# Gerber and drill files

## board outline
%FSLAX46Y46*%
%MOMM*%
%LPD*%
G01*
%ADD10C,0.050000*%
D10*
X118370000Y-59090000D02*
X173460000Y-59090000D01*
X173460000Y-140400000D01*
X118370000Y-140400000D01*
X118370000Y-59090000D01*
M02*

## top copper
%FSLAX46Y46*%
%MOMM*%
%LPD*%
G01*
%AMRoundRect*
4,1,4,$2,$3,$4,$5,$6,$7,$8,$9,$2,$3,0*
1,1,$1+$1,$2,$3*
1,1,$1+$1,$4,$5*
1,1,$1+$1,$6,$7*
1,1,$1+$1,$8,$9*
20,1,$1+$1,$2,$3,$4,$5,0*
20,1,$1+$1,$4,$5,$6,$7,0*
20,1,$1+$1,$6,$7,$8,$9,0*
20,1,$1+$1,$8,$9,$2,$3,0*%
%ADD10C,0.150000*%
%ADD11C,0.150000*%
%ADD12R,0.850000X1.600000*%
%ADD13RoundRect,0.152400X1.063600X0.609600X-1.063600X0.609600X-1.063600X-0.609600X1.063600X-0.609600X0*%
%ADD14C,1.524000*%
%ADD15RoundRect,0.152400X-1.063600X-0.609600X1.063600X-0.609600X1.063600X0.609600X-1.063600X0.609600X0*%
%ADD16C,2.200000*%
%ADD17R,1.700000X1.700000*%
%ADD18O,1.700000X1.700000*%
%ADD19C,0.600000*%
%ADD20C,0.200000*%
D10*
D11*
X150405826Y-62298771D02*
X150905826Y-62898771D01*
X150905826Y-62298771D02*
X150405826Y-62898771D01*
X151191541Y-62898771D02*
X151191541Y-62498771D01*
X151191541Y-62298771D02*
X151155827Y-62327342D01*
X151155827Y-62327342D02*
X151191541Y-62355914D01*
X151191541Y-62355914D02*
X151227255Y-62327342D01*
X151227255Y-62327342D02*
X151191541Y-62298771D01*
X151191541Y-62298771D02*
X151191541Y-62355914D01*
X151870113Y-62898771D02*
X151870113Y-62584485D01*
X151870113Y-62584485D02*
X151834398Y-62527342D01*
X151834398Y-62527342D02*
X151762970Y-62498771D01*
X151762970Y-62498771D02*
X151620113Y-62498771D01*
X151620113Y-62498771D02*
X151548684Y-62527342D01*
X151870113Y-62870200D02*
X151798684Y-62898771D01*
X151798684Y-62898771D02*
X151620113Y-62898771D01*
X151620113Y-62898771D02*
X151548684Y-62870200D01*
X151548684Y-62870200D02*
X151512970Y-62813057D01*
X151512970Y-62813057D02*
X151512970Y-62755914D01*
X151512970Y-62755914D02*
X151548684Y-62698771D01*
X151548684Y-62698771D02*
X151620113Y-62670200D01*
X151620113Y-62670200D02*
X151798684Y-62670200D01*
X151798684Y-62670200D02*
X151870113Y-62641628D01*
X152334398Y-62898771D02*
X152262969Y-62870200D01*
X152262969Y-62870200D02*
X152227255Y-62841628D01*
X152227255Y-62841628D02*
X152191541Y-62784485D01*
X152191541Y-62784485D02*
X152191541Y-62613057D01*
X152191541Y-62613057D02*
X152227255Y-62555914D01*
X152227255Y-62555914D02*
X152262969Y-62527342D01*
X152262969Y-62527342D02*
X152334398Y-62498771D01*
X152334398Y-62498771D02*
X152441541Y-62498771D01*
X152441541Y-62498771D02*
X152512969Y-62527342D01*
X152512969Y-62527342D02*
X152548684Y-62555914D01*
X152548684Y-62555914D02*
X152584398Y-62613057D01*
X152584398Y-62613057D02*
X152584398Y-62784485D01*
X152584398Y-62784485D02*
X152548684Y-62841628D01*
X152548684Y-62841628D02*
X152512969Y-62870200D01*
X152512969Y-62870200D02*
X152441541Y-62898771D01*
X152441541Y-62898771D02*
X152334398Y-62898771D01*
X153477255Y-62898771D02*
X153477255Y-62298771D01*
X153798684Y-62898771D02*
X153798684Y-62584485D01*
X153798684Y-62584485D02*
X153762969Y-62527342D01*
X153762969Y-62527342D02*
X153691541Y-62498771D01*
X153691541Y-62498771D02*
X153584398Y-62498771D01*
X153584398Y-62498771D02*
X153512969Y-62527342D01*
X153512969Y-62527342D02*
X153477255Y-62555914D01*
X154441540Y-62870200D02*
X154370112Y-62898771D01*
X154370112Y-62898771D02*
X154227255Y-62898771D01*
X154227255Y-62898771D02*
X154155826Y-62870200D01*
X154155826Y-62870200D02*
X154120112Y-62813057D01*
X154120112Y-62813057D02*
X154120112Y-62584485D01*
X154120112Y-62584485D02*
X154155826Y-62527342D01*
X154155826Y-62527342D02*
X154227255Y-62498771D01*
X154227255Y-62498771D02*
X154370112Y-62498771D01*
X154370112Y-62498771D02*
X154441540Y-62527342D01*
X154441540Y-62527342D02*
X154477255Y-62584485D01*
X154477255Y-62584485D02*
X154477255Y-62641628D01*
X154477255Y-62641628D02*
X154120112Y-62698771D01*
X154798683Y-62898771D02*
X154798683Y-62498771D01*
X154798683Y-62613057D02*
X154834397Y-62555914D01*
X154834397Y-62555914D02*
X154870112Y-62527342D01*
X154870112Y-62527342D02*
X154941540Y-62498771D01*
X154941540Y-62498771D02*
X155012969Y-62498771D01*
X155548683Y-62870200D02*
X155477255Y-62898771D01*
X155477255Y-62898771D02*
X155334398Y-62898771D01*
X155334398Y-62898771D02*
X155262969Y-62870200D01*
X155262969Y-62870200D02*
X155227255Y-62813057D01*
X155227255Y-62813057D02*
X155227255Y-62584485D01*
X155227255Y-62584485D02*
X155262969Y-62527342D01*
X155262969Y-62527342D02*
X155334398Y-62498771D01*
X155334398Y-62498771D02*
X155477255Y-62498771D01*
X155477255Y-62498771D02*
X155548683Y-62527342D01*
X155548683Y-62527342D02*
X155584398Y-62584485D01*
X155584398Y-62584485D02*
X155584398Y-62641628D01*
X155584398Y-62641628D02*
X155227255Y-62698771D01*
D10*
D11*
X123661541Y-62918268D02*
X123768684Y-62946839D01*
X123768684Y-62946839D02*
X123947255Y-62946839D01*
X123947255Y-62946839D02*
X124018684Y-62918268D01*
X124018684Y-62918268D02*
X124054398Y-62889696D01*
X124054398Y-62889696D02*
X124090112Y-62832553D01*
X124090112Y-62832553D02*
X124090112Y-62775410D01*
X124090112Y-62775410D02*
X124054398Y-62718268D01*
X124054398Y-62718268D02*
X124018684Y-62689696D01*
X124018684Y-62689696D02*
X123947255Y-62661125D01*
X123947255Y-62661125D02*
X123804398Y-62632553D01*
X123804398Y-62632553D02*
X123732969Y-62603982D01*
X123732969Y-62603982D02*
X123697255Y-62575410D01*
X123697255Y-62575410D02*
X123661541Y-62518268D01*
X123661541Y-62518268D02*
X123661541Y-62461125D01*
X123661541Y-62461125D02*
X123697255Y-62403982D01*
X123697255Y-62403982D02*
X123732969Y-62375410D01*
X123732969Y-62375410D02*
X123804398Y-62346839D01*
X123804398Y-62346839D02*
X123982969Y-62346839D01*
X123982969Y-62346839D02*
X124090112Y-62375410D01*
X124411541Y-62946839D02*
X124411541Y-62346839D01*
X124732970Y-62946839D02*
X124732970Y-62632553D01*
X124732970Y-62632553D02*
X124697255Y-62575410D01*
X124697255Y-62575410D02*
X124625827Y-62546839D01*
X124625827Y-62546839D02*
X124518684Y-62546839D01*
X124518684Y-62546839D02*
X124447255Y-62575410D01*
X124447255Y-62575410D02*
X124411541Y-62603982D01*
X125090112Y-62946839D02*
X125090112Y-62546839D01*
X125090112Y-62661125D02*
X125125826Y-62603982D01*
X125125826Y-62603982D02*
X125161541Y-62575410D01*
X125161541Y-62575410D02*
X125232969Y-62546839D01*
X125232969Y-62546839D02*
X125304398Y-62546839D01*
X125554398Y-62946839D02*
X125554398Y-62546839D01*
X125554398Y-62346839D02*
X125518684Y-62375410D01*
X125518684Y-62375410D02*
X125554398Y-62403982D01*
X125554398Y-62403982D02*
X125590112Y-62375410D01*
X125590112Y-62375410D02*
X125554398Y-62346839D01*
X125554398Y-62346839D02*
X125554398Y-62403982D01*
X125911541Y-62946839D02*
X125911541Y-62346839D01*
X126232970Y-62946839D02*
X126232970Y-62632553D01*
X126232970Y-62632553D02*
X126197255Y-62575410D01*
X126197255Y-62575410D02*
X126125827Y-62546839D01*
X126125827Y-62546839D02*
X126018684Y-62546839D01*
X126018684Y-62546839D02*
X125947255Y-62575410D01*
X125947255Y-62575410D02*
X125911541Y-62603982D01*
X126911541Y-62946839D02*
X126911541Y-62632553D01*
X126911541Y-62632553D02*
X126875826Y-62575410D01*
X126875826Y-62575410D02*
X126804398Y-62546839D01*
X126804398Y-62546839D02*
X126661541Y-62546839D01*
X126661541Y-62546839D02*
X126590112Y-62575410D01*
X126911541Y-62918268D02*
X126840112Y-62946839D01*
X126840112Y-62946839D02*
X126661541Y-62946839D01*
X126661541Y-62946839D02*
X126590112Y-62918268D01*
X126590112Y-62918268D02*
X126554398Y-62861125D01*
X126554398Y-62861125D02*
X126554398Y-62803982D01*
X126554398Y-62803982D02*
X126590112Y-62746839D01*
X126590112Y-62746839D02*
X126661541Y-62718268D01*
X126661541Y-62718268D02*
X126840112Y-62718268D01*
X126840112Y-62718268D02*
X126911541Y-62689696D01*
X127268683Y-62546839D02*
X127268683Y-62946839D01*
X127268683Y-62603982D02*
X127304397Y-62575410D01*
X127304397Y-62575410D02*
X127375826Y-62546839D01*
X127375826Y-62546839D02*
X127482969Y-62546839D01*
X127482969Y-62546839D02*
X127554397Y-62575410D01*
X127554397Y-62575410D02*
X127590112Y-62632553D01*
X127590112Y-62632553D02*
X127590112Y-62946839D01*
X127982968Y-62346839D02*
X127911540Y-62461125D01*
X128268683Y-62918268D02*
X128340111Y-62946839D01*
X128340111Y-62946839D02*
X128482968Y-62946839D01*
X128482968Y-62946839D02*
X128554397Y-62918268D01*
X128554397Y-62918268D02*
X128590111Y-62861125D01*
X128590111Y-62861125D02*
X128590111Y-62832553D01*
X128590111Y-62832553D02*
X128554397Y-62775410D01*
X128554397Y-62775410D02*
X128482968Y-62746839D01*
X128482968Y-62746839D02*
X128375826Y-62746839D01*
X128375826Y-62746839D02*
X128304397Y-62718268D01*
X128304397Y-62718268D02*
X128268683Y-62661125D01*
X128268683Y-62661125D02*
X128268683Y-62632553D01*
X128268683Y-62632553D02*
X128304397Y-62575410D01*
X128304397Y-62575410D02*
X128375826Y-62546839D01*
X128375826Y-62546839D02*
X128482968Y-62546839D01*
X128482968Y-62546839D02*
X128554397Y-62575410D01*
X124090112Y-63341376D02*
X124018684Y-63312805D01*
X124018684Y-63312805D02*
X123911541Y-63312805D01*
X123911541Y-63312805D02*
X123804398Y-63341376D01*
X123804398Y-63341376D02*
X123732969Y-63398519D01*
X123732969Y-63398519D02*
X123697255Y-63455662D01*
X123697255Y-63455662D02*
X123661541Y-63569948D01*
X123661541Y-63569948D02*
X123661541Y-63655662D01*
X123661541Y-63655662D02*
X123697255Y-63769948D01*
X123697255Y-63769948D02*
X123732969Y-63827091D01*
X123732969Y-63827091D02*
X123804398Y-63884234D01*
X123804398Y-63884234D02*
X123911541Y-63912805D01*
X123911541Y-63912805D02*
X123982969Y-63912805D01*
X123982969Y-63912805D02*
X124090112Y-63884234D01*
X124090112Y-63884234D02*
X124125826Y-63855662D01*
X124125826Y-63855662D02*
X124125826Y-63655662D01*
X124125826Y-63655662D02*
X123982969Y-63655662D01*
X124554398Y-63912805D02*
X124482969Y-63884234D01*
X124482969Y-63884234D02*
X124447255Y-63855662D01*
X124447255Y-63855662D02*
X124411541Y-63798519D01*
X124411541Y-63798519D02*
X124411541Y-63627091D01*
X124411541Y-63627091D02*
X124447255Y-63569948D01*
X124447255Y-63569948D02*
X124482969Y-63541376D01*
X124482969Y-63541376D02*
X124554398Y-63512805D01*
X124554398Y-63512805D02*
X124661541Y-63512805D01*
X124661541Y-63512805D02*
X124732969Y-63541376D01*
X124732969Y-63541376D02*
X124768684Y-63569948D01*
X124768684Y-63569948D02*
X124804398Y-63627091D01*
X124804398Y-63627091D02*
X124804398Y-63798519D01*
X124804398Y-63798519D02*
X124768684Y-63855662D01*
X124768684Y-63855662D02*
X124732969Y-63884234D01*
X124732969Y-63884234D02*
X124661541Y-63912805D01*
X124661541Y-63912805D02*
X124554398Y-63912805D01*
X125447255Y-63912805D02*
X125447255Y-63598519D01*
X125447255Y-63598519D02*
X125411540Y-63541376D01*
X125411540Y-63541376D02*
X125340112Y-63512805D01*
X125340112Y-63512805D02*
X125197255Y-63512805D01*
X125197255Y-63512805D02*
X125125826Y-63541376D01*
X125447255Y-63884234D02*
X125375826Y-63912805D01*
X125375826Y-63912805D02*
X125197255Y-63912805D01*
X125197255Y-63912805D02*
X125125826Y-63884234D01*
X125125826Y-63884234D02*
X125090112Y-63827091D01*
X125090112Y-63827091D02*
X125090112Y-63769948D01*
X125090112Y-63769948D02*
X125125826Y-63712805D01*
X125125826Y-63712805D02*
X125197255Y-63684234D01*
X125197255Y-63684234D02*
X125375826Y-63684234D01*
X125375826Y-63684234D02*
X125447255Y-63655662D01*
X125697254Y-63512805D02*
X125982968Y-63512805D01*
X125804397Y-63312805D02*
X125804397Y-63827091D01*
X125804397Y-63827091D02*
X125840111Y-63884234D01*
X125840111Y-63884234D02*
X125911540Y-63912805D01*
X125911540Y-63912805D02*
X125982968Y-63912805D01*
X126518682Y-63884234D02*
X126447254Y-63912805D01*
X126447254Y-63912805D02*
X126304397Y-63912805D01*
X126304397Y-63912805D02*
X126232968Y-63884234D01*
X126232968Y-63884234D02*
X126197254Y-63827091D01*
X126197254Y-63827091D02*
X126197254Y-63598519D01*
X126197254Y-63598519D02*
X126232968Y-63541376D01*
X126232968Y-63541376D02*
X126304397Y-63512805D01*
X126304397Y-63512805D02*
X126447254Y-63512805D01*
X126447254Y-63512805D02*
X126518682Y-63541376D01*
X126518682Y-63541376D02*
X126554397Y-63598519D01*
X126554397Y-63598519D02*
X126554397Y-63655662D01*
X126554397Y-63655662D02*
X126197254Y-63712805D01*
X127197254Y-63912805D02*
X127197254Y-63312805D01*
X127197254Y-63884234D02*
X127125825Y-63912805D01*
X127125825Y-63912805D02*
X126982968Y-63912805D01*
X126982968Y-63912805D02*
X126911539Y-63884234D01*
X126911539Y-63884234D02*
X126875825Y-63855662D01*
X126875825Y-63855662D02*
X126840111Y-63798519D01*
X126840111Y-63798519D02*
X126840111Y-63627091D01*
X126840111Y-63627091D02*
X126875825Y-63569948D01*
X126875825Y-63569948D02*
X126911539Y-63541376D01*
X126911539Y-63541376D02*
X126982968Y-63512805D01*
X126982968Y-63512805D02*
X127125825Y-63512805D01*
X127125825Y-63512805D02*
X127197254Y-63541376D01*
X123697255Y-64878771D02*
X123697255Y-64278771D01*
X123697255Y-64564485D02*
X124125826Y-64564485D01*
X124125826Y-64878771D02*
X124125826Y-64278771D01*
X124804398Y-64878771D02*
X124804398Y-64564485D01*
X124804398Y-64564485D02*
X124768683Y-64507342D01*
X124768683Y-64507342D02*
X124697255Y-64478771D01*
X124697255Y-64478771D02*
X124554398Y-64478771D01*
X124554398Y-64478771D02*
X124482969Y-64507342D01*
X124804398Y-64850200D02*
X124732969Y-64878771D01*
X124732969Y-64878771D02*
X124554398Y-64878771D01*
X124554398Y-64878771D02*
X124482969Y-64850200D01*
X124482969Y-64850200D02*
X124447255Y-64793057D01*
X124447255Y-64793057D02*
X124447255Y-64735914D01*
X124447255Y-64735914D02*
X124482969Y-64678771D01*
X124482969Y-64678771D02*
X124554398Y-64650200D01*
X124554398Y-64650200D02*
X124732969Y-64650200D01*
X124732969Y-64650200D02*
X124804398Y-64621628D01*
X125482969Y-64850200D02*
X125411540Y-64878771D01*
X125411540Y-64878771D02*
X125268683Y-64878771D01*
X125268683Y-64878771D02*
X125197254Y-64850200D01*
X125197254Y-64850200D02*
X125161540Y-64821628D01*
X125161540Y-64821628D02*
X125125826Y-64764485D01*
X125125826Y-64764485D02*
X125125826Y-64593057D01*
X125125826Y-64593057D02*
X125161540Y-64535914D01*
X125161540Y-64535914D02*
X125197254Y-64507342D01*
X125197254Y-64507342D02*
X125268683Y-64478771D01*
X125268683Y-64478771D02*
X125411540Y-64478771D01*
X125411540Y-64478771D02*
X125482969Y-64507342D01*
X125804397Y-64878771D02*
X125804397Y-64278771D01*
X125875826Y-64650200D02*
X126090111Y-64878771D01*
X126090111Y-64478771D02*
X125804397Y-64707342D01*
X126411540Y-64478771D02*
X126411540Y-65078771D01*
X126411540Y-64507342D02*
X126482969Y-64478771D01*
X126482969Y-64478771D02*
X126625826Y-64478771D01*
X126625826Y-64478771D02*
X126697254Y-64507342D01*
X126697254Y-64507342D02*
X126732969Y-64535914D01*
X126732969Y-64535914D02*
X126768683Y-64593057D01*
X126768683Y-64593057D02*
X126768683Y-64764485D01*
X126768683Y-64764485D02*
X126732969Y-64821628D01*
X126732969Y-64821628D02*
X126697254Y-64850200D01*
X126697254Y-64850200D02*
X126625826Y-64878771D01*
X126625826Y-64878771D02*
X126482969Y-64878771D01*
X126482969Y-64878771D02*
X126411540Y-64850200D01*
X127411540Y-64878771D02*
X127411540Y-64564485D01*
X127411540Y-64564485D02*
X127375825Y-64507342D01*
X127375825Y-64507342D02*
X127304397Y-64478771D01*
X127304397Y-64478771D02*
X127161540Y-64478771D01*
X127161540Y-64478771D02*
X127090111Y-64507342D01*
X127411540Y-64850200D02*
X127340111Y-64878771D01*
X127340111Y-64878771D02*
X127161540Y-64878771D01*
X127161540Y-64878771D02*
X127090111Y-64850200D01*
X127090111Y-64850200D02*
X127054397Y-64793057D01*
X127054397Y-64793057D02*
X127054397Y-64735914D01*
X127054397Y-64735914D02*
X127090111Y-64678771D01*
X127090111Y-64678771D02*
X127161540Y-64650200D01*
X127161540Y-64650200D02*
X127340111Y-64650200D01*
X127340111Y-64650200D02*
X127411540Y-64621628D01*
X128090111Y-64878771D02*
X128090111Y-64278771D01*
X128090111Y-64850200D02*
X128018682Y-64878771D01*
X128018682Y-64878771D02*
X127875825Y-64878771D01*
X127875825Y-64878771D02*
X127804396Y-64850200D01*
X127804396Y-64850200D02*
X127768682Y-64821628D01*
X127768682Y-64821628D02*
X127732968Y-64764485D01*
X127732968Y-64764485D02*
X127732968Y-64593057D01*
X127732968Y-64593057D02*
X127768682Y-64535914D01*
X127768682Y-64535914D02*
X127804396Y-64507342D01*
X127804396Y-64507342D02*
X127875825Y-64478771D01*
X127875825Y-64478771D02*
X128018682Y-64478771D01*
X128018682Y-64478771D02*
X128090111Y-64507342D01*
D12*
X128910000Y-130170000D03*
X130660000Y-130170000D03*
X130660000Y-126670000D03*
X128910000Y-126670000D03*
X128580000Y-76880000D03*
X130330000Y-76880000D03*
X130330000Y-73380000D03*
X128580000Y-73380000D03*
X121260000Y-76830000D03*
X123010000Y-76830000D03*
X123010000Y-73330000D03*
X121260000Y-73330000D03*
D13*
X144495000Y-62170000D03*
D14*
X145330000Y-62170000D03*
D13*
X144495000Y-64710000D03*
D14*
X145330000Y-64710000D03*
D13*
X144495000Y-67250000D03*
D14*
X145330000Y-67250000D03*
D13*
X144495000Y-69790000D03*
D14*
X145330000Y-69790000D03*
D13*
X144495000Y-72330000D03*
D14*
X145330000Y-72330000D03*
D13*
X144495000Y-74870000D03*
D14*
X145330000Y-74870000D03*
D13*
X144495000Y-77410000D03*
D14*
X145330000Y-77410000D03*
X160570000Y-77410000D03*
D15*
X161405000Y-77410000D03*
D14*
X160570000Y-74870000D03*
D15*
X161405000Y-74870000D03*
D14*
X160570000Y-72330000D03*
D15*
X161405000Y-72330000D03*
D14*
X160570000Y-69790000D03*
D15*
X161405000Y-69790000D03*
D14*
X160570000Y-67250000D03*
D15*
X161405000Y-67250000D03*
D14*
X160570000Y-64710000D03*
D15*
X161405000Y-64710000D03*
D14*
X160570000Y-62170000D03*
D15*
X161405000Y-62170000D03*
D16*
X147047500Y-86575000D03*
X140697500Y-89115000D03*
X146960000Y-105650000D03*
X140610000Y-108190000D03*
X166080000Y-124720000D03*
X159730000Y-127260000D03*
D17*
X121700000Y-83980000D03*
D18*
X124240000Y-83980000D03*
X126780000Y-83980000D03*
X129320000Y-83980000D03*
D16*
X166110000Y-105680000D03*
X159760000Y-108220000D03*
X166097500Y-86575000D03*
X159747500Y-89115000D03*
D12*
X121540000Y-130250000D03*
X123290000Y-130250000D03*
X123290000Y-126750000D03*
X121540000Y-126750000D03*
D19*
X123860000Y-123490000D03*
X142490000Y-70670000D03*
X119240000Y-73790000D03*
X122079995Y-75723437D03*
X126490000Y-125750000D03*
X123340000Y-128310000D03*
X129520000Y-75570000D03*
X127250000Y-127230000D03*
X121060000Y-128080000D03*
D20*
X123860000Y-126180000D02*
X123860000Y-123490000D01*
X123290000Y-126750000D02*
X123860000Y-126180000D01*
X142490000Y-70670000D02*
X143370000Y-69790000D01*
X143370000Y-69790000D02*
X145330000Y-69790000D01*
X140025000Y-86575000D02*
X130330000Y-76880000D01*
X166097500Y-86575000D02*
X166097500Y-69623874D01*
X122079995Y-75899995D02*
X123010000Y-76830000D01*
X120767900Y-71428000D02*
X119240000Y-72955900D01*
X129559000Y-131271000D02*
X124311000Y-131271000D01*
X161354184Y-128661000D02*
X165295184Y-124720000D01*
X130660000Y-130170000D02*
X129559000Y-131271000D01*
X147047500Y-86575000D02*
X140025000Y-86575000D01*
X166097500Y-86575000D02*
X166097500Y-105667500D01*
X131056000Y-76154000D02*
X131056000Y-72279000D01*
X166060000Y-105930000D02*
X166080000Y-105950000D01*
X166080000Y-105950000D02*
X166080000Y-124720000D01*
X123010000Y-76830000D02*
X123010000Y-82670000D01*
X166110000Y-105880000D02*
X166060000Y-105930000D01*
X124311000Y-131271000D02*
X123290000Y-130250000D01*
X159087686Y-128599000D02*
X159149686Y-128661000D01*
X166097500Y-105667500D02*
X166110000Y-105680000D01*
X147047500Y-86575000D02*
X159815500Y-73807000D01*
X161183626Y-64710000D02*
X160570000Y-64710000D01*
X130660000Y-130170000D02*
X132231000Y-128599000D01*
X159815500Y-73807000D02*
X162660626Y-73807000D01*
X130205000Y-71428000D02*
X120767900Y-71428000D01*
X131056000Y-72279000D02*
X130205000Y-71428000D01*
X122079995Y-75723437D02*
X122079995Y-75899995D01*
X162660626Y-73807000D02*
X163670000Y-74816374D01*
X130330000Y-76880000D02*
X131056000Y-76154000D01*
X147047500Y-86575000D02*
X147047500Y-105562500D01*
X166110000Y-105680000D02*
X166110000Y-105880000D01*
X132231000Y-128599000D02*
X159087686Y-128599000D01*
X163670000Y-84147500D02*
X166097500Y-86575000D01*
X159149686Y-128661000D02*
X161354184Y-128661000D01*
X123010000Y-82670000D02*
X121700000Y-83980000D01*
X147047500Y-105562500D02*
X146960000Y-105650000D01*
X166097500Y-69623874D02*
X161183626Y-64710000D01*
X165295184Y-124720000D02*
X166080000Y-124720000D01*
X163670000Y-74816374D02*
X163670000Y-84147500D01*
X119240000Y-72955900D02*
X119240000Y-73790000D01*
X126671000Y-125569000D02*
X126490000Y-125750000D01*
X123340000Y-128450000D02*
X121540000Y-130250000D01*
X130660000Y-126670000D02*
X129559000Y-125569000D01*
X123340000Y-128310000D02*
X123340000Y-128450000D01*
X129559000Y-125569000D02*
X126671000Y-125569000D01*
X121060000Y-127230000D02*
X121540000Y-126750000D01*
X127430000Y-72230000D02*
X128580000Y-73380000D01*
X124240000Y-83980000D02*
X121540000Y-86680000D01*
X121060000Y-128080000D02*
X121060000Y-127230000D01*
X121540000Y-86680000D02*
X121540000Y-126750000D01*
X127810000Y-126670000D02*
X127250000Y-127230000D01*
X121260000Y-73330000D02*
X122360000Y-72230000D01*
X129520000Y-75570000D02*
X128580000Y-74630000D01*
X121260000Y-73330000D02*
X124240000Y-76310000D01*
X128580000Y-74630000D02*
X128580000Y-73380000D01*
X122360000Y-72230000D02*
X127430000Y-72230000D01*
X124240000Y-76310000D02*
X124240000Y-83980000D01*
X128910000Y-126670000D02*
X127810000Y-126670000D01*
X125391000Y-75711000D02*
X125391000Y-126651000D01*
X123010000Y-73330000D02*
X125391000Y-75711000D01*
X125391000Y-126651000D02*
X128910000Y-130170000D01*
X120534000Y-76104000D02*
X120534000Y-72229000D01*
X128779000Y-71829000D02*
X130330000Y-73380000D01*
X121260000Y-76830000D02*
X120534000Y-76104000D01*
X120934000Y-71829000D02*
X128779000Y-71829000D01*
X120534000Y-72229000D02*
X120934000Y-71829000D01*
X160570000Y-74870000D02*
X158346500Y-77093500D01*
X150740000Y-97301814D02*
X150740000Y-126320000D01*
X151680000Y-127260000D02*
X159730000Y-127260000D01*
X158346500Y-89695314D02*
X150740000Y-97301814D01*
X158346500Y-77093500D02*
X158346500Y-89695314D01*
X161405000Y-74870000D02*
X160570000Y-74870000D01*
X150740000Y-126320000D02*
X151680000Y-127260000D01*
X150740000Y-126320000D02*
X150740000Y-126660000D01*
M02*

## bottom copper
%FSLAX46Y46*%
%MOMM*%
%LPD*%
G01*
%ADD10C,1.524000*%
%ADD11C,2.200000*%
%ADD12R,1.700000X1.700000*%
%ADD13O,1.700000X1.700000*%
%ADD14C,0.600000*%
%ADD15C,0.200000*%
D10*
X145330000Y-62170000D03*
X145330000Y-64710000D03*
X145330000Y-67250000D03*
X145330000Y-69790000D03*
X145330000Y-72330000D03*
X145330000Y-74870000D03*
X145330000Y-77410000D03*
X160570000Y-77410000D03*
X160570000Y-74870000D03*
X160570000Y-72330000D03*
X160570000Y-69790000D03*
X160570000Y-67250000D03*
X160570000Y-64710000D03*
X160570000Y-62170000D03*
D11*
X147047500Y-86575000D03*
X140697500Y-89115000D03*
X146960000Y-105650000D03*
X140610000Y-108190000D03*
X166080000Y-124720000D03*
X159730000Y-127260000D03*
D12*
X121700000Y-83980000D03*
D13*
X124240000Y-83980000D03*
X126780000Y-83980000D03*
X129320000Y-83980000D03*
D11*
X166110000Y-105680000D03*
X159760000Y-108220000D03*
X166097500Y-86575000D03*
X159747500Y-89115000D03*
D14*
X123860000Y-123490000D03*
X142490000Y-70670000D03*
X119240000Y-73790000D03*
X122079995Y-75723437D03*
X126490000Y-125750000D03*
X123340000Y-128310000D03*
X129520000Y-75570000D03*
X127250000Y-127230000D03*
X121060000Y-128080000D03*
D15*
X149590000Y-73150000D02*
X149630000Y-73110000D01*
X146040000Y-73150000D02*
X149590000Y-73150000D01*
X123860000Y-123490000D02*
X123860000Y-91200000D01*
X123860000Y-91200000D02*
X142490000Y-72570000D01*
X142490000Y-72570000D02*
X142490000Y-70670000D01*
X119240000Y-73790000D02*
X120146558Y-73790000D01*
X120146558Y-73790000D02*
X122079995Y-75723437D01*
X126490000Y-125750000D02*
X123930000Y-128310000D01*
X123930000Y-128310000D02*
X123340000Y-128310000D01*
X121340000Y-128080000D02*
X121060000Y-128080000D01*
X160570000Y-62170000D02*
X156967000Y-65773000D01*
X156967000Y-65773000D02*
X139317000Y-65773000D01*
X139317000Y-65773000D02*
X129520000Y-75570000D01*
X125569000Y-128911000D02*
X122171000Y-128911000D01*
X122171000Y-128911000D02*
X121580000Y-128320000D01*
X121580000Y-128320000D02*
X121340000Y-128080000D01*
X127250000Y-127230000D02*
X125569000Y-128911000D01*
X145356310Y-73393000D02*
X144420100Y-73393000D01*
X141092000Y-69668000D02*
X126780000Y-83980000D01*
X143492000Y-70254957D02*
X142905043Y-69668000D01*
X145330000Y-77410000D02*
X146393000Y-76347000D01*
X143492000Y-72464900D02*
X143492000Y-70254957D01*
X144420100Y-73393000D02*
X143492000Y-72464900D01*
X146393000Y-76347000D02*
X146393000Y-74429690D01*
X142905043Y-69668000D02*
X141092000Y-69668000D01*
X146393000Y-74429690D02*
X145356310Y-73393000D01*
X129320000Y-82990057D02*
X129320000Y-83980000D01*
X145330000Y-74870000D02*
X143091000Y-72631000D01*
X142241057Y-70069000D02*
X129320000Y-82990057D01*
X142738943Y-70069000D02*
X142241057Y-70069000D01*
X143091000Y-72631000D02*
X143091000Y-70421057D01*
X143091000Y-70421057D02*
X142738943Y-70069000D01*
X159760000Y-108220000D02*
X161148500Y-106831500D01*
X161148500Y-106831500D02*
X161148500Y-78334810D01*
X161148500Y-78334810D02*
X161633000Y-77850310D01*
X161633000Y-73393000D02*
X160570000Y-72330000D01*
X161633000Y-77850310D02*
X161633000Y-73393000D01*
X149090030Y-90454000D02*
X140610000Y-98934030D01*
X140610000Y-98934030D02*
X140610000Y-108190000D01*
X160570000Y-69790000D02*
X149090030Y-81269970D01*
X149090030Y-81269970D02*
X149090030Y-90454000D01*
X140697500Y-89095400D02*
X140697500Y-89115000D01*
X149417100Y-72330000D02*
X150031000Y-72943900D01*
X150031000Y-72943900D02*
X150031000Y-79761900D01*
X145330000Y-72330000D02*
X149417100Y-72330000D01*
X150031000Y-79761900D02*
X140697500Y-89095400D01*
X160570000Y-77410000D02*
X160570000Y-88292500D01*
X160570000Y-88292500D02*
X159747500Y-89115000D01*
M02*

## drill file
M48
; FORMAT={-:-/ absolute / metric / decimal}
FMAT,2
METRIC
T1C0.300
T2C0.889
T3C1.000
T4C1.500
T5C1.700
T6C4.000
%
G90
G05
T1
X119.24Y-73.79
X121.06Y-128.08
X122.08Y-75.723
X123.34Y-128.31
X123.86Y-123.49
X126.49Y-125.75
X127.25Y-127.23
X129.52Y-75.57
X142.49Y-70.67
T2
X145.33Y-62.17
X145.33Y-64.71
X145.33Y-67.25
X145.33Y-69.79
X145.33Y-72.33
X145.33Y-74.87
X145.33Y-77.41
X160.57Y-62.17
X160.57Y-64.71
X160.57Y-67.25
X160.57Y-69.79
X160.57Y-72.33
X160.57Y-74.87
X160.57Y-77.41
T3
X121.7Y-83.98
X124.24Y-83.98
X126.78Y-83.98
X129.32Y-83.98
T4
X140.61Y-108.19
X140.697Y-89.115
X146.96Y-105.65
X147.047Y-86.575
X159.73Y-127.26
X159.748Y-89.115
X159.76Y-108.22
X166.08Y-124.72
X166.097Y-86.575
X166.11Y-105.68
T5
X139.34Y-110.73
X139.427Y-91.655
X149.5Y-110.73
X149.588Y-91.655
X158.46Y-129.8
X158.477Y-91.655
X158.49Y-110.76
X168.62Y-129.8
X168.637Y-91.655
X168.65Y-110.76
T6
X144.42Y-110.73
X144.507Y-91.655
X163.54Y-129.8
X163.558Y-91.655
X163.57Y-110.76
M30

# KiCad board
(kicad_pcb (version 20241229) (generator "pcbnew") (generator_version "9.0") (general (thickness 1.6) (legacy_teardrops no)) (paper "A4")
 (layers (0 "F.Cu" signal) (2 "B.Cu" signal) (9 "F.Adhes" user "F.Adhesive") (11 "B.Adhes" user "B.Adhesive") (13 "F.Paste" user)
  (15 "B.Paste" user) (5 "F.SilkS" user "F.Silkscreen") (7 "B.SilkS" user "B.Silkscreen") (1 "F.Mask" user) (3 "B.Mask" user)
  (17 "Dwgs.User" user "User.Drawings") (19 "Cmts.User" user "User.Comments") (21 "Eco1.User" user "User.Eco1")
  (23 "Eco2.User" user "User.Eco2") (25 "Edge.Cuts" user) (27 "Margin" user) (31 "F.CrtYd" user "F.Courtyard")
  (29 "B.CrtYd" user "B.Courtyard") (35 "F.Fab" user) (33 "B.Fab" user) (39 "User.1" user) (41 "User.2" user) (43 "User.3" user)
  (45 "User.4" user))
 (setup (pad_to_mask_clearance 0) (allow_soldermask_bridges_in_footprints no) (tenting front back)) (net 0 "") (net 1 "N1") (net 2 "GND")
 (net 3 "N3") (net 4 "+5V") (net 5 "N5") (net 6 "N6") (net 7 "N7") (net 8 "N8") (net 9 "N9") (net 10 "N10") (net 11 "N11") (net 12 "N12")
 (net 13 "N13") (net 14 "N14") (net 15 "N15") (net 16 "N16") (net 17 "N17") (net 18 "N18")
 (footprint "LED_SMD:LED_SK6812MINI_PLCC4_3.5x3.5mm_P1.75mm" (layer "F.Cu") (at 129.785 128.42 90)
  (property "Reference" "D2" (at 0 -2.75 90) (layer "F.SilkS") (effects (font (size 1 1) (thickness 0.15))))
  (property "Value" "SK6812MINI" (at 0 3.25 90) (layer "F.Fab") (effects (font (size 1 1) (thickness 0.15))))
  (pad "1" smd rect (at -1.75 -0.875 90) (size 1.6 0.85) (layers "F.Cu" "F.Mask" "F.Paste") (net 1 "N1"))
  (pad "2" smd rect (at -1.75 0.875 90) (size 1.6 0.85) (layers "F.Cu" "F.Mask" "F.Paste") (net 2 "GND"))
  (pad "3" smd rect (at 1.75 0.875 90) (size 1.6 0.85) (layers "F.Cu" "F.Mask" "F.Paste") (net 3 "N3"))
  (pad "4" smd rect (at 1.75 -0.875 90) (size 1.6 0.85) (layers "F.Cu" "F.Mask" "F.Paste") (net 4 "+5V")))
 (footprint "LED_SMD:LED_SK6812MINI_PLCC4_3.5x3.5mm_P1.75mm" (layer "F.Cu") (at 129.455 75.13 90)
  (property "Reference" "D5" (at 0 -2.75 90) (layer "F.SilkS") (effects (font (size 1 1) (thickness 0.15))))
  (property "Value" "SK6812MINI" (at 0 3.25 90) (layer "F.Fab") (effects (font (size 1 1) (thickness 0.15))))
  (pad "1" smd rect (at -1.75 -0.875 90) (size 1.6 0.85) (layers "F.Cu" "F.Mask" "F.Paste") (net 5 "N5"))
  (pad "2" smd rect (at -1.75 0.875 90) (size 1.6 0.85) (layers "F.Cu" "F.Mask" "F.Paste") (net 2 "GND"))
  (pad "3" smd rect (at 1.75 0.875 90) (size 1.6 0.85) (layers "F.Cu" "F.Mask" "F.Paste") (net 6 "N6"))
  (pad "4" smd rect (at 1.75 -0.875 90) (size 1.6 0.85) (layers "F.Cu" "F.Mask" "F.Paste") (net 4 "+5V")))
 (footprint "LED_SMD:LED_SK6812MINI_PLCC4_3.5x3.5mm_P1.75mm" (layer "F.Cu") (at 122.135 75.08 90)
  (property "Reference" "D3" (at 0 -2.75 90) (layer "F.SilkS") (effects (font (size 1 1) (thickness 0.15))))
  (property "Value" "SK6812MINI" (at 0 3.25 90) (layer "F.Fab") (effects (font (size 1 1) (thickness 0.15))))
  (pad "1" smd rect (at -1.75 -0.875 90) (size 1.6 0.85) (layers "F.Cu" "F.Mask" "F.Paste") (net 6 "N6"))
  (pad "2" smd rect (at -1.75 0.875 90) (size 1.6 0.85) (layers "F.Cu" "F.Mask" "F.Paste") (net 2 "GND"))
  (pad "3" smd rect (at 1.75 0.875 90) (size 1.6 0.85) (layers "F.Cu" "F.Mask" "F.Paste") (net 1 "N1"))
  (pad "4" smd rect (at 1.75 -0.875 90) (size 1.6 0.85) (layers "F.Cu" "F.Mask" "F.Paste") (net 4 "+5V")))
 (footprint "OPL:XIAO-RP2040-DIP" (layer "F.Cu") (at 152.95 69.79)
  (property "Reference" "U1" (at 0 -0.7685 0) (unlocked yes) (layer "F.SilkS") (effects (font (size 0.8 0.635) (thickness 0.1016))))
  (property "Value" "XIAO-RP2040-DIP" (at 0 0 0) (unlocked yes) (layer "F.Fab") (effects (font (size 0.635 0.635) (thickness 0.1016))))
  (pad "1" smd roundrect (at -8.455 -7.62 180) (size 2.432 1.524) (layers "F.Cu" "F.Mask") (roundrect_rratio 0.1) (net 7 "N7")
   (thermal_bridge_angle 45))
  (pad "1" thru_hole circle (at -7.62 -7.62 180) (size 1.524 1.524) (drill 0.889) (layers "*.Cu" "*.Mask") (remove_unused_layers no)
   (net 7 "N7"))
  (pad "2" smd roundrect (at -8.455 -5.08 180) (size 2.432 1.524) (layers "F.Cu" "F.Mask") (roundrect_rratio 0.1) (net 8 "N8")
   (thermal_bridge_angle 45))
  (pad "2" thru_hole circle (at -7.62 -5.08 180) (size 1.524 1.524) (drill 0.889) (layers "*.Cu" "*.Mask") (remove_unused_layers no)
   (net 8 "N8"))
  (pad "3" smd roundrect (at -8.455 -2.54 180) (size 2.432 1.524) (layers "F.Cu" "F.Mask") (roundrect_rratio 0.1) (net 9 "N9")
   (thermal_bridge_angle 45))
  (pad "3" thru_hole circle (at -7.62 -2.54 180) (size 1.524 1.524) (drill 0.889) (layers "*.Cu" "*.Mask") (remove_unused_layers no)
   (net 9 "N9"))
  (pad "4" smd roundrect (at -8.455 0 180) (size 2.432 1.524) (layers "F.Cu" "F.Mask") (roundrect_rratio 0.1) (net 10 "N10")
   (thermal_bridge_angle 45))
  (pad "4" thru_hole circle (at -7.62 0 180) (size 1.524 1.524) (drill 0.889) (layers "*.Cu" "*.Mask") (remove_unused_layers no)
   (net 10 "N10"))
  (pad "5" smd roundrect (at -8.455 2.54 180) (size 2.432 1.524) (layers "F.Cu" "F.Mask") (roundrect_rratio 0.1) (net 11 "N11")
   (thermal_bridge_angle 45))
  (pad "5" thru_hole circle (at -7.62 2.54 180) (size 1.524 1.524) (drill 0.889) (layers "*.Cu" "*.Mask") (remove_unused_layers no)
   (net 11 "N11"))
  (pad "6" smd roundrect (at -8.455 5.08 180) (size 2.432 1.524) (layers "F.Cu" "F.Mask") (roundrect_rratio 0.1) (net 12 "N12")
   (thermal_bridge_angle 45))
  (pad "6" thru_hole circle (at -7.62 5.08 180) (size 1.524 1.524) (drill 0.889) (layers "*.Cu" "*.Mask") (remove_unused_layers no)
   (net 12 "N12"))
  (pad "7" smd roundrect (at -8.455 7.62 180) (size 2.432 1.524) (layers "F.Cu" "F.Mask") (roundrect_rratio 0.1) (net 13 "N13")
   (thermal_bridge_angle 45))
  (pad "7" thru_hole circle (at -7.62 7.62 180) (size 1.524 1.524) (drill 0.889) (layers "*.Cu" "*.Mask") (remove_unused_layers no)
   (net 13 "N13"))
  (pad "8" thru_hole circle (at 7.62 7.62) (size 1.524 1.524) (drill 0.889) (layers "*.Cu" "*.Mask") (remove_unused_layers no)
   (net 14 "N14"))
  (pad "8" smd roundrect (at 8.455 7.62) (size 2.432 1.524) (layers "F.Cu" "F.Mask") (roundrect_rratio 0.1) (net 14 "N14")
   (thermal_bridge_angle 45))
  (pad "9" thru_hole circle (at 7.62 5.08) (size 1.524 1.524) (drill 0.889) (layers "*.Cu" "*.Mask") (remove_unused_layers no)
   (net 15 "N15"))
  (pad "9" smd roundrect (at 8.455 5.08) (size 2.432 1.524) (layers "F.Cu" "F.Mask") (roundrect_rratio 0.1) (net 15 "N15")
   (thermal_bridge_angle 45))
  (pad "10" thru_hole circle (at 7.62 2.54) (size 1.524 1.524) (drill 0.889) (layers "*.Cu" "*.Mask") (remove_unused_layers no)
   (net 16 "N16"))
  (pad "10" smd roundrect (at 8.455 2.54) (size 2.432 1.524) (layers "F.Cu" "F.Mask") (roundrect_rratio 0.1) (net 16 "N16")
   (thermal_bridge_angle 45))
  (pad "11" thru_hole circle (at 7.62 0) (size 1.524 1.524) (drill 0.889) (layers "*.Cu" "*.Mask") (remove_unused_layers no) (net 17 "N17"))
  (pad "11" smd roundrect (at 8.455 0) (size 2.432 1.524) (layers "F.Cu" "F.Mask") (roundrect_rratio 0.1) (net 17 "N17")
   (thermal_bridge_angle 45))
  (pad "12" thru_hole circle (at 7.62 -2.54) (size 1.524 1.524) (drill 0.889) (layers "*.Cu" "*.Mask") (remove_unused_layers no)
   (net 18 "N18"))
  (pad "12" smd roundrect (at 8.455 -2.54) (size 2.432 1.524) (layers "F.Cu" "F.Mask") (roundrect_rratio 0.1) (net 18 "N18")
   (thermal_bridge_angle 45))
  (pad "13" thru_hole circle (at 7.62 -5.08) (size 1.524 1.524) (drill 0.889) (layers "*.Cu" "*.Mask") (remove_unused_layers no)
   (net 2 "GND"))
  (pad "13" smd roundrect (at 8.455 -5.08) (size 2.432 1.524) (layers "F.Cu" "F.Mask") (roundrect_rratio 0.1) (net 2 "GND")
   (thermal_bridge_angle 45))
  (pad "14" thru_hole circle (at 7.62 -7.62) (size 1.524 1.524) (drill 0.889) (layers "*.Cu" "*.Mask") (remove_unused_layers no)
   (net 4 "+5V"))
  (pad "14" smd roundrect (at 8.455 -7.62) (size 2.432 1.524) (layers "F.Cu" "F.Mask") (roundrect_rratio 0.1) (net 4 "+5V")
   (thermal_bridge_angle 45)))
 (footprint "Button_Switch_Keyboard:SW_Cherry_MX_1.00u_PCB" (layer "F.Cu") (at 147.0475 86.575)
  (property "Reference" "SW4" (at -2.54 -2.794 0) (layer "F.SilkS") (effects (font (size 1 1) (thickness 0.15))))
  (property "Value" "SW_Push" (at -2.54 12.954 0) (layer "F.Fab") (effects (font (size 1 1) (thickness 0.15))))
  (pad "" np_thru_hole circle (at -7.62 5.08) (size 1.7 1.7) (drill 1.7) (layers "*.Cu" "*.Mask"))
  (pad "" np_thru_hole circle (at -2.54 5.08) (size 4 4) (drill 4) (layers "*.Cu" "*.Mask"))
  (pad "" np_thru_hole circle (at 2.54 5.08) (size 1.7 1.7) (drill 1.7) (layers "*.Cu" "*.Mask"))
  (pad "1" thru_hole circle (at 0 0) (size 2.2 2.2) (drill 1.5) (layers "*.Cu" "*.Mask") (remove_unused_layers no) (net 2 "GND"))
  (pad "2" thru_hole circle (at -6.35 2.54) (size 2.2 2.2) (drill 1.5) (layers "*.Cu" "*.Mask") (remove_unused_layers no) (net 11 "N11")))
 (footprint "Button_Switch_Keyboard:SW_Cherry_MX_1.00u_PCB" (layer "F.Cu") (at 146.96 105.65)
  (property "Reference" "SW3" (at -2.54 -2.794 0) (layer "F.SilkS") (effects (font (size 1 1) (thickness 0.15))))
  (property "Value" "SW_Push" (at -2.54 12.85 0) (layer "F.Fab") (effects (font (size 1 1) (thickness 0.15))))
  (pad "" np_thru_hole circle (at -7.62 5.08) (size 1.7 1.7) (drill 1.7) (layers "*.Cu" "*.Mask"))
  (pad "" np_thru_hole circle (at -2.54 5.08) (size 4 4) (drill 4) (layers "*.Cu" "*.Mask"))
  (pad "" np_thru_hole circle (at 2.54 5.08) (size 1.7 1.7) (drill 1.7) (layers "*.Cu" "*.Mask"))
  (pad "1" thru_hole circle (at 0 0) (size 2.2 2.2) (drill 1.5) (layers "*.Cu" "*.Mask") (remove_unused_layers no) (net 2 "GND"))
  (pad "2" thru_hole circle (at -6.35 2.54) (size 2.2 2.2) (drill 1.5) (layers "*.Cu" "*.Mask") (remove_unused_layers no) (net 17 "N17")))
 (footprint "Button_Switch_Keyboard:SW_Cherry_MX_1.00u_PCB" (layer "F.Cu") (at 166.08 124.72)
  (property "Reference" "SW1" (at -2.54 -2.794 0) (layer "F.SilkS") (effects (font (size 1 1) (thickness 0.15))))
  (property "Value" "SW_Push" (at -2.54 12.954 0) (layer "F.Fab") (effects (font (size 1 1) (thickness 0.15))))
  (pad "" np_thru_hole circle (at -7.62 5.08) (size 1.7 1.7) (drill 1.7) (layers "*.Cu" "*.Mask"))
  (pad "" np_thru_hole circle (at -2.54 5.08) (size 4 4) (drill 4) (layers "*.Cu" "*.Mask"))
  (pad "" np_thru_hole circle (at 2.54 5.08) (size 1.7 1.7) (drill 1.7) (layers "*.Cu" "*.Mask"))
  (pad "1" thru_hole circle (at 0 0) (size 2.2 2.2) (drill 1.5) (layers "*.Cu" "*.Mask") (remove_unused_layers no) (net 2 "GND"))
  (pad "2" thru_hole circle (at -6.35 2.54) (size 2.2 2.2) (drill 1.5) (layers "*.Cu" "*.Mask") (remove_unused_layers no) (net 15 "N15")))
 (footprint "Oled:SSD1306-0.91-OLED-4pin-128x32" (layer "F.Cu") (at 119.51 120.48 90)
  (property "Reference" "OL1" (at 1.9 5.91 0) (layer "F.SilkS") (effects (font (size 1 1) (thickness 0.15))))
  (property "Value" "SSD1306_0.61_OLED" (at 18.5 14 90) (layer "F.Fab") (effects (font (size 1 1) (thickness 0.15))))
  (pad "1" thru_hole rect (at 36.5 2.19 90) (size 1.7 1.7) (drill 1) (layers "*.Cu" "*.Mask") (remove_unused_layers no) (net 2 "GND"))
  (pad "2" thru_hole oval (at 36.5 4.73 90) (size 1.7 1.7) (drill 1) (layers "*.Cu" "*.Mask") (remove_unused_layers no) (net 4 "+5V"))
  (pad "3" thru_hole oval (at 36.5 7.27 90) (size 1.7 1.7) (drill 1) (layers "*.Cu" "*.Mask") (remove_unused_layers no) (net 13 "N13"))
  (pad "4" thru_hole oval (at 36.5 9.81 90) (size 1.7 1.7) (drill 1) (layers "*.Cu" "*.Mask") (remove_unused_layers no) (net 12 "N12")))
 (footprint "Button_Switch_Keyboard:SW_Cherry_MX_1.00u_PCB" (layer "F.Cu") (at 166.11 105.68)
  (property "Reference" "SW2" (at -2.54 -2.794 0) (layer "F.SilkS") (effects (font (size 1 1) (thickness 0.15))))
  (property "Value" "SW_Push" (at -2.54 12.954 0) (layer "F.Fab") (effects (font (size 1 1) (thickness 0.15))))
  (pad "" np_thru_hole circle (at -7.62 5.08) (size 1.7 1.7) (drill 1.7) (layers "*.Cu" "*.Mask"))
  (pad "" np_thru_hole circle (at -2.54 5.08) (size 4 4) (drill 4) (layers "*.Cu" "*.Mask"))
  (pad "" np_thru_hole circle (at 2.54 5.08) (size 1.7 1.7) (drill 1.7) (layers "*.Cu" "*.Mask"))
  (pad "1" thru_hole circle (at 0 0) (size 2.2 2.2) (drill 1.5) (layers "*.Cu" "*.Mask") (remove_unused_layers no) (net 2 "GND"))
  (pad "2" thru_hole circle (at -6.35 2.54) (size 2.2 2.2) (drill 1.5) (layers "*.Cu" "*.Mask") (remove_unused_layers no) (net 16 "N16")))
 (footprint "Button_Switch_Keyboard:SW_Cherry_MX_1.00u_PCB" (layer "F.Cu") (at 166.0975 86.575)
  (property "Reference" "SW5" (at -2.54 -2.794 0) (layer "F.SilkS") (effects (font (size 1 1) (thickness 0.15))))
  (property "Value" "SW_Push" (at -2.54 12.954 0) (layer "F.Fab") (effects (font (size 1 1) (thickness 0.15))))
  (pad "" np_thru_hole circle (at -7.62 5.08) (size 1.7 1.7) (drill 1.7) (layers "*.Cu" "*.Mask"))
  (pad "" np_thru_hole circle (at -2.54 5.08) (size 4 4) (drill 4) (layers "*.Cu" "*.Mask"))
  (pad "" np_thru_hole circle (at 2.54 5.08) (size 1.7 1.7) (drill 1.7) (layers "*.Cu" "*.Mask"))
  (pad "1" thru_hole circle (at 0 0) (size 2.2 2.2) (drill 1.5) (layers "*.Cu" "*.Mask") (remove_unused_layers no) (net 2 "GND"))
  (pad "2" thru_hole circle (at -6.35 2.54) (size 2.2 2.2) (drill 1.5) (layers "*.Cu" "*.Mask") (remove_unused_layers no) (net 14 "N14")))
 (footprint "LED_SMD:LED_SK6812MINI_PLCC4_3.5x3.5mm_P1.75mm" (layer "F.Cu") (at 122.415 128.5 90)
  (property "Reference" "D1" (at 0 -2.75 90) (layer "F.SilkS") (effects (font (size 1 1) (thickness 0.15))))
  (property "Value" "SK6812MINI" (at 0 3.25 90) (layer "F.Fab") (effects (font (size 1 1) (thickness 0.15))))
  (pad "1" smd rect (at -1.75 -0.875 90) (size 1.6 0.85) (layers "F.Cu" "F.Mask" "F.Paste") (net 3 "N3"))
  (pad "2" smd rect (at -1.75 0.875 90) (size 1.6 0.85) (layers "F.Cu" "F.Mask" "F.Paste") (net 2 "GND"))
  (pad "3" smd rect (at 1.75 0.875 90) (size 1.6 0.85) (layers "F.Cu" "F.Mask" "F.Paste") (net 10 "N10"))
  (pad "4" smd rect (at 1.75 -0.875 90) (size 1.6 0.85) (layers "F.Cu" "F.Mask" "F.Paste") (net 4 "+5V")))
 (gr_rect (start 118.37 59.09) (end 173.46 140.4) (stroke (width 0.05) (type default)) (fill no) (layer "Edge.Cuts"))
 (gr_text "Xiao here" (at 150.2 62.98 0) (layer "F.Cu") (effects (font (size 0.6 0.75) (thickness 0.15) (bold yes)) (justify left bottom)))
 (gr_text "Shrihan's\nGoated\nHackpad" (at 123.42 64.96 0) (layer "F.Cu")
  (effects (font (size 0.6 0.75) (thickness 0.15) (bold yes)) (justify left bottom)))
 (segment (start 149.59 73.15) (end 149.63 73.11) (width 0.2) (layer "B.Cu") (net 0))
 (segment (start 146.04 73.15) (end 149.59 73.15) (width 0.2) (layer "B.Cu") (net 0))
 (segment (start 123.86 126.18) (end 123.86 123.49) (width 0.2) (layer "F.Cu") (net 10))
 (segment (start 123.29 126.75) (end 123.86 126.18) (width 0.2) (layer "F.Cu") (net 10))
 (segment (start 142.49 70.67) (end 143.37 69.79) (width 0.2) (layer "F.Cu") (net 10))
 (segment (start 143.37 69.79) (end 145.33 69.79) (width 0.2) (layer "F.Cu") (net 10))
 (via (at 123.86 123.49) (size 0.6) (drill 0.3) (layers "F.Cu" "B.Cu") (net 10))
 (via (at 142.49 70.67) (size 0.6) (drill 0.3) (layers "F.Cu" "B.Cu") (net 10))
 (segment (start 123.86 123.49) (end 123.86 91.2) (width 0.2) (layer "B.Cu") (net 10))
 (segment (start 123.86 91.2) (end 142.49 72.57) (width 0.2) (layer "B.Cu") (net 10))
 (segment (start 142.49 72.57) (end 142.49 70.67) (width 0.2) (layer "B.Cu") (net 10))
 (segment (start 140.025 86.575) (end 130.33 76.88) (width 0.2) (layer "F.Cu") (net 2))
 (segment (start 166.0975 86.575) (end 166.0975 69.623874) (width 0.2) (layer "F.Cu") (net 2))
 (segment (start 122.079995 75.899995) (end 123.01 76.83) (width 0.2) (layer "F.Cu") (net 2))
 (segment (start 120.7679 71.428) (end 119.24 72.9559) (width 0.2) (layer "F.Cu") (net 2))
 (segment (start 129.559 131.271) (end 124.311 131.271) (width 0.2) (layer "F.Cu") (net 2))
 (segment (start 161.354184 128.661) (end 165.295184 124.72) (width 0.2) (layer "F.Cu") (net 2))
 (segment (start 130.66 130.17) (end 129.559 131.271) (width 0.2) (layer "F.Cu") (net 2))
 (segment (start 147.0475 86.575) (end 140.025 86.575) (width 0.2) (layer "F.Cu") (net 2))
 (segment (start 166.0975 86.575) (end 166.0975 105.6675) (width 0.2) (layer "F.Cu") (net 2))
 (segment (start 131.056 76.154) (end 131.056 72.279) (width 0.2) (layer "F.Cu") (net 2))
 (segment (start 166.06 105.93) (end 166.08 105.95) (width 0.2) (layer "F.Cu") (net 2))
 (segment (start 166.08 105.95) (end 166.08 124.72) (width 0.2) (layer "F.Cu") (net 2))
 (segment (start 123.01 76.83) (end 123.01 82.67) (width 0.2) (layer "F.Cu") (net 2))
 (segment (start 166.11 105.88) (end 166.06 105.93) (width 0.2) (layer "F.Cu") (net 2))
 (segment (start 124.311 131.271) (end 123.29 130.25) (width 0.2) (layer "F.Cu") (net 2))
 (segment (start 159.087686 128.599) (end 159.149686 128.661) (width 0.2) (layer "F.Cu") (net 2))
 (segment (start 166.0975 105.6675) (end 166.11 105.68) (width 0.2) (layer "F.Cu") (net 2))
 (segment (start 147.0475 86.575) (end 159.8155 73.807) (width 0.2) (layer "F.Cu") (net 2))
 (segment (start 161.183626 64.71) (end 160.57 64.71) (width 0.2) (layer "F.Cu") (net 2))
 (segment (start 130.66 130.17) (end 132.231 128.599) (width 0.2) (layer "F.Cu") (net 2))
 (segment (start 159.8155 73.807) (end 162.660626 73.807) (width 0.2) (layer "F.Cu") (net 2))
 (segment (start 130.205 71.428) (end 120.7679 71.428) (width 0.2) (layer "F.Cu") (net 2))
 (segment (start 131.056 72.279) (end 130.205 71.428) (width 0.2) (layer "F.Cu") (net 2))
 (segment (start 122.079995 75.723437) (end 122.079995 75.899995) (width 0.2) (layer "F.Cu") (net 2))
 (segment (start 162.660626 73.807) (end 163.67 74.816374) (width 0.2) (layer "F.Cu") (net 2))
 (segment (start 130.33 76.88) (end 131.056 76.154) (width 0.2) (layer "F.Cu") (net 2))
 (segment (start 147.0475 86.575) (end 147.0475 105.5625) (width 0.2) (layer "F.Cu") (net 2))
 (segment (start 166.11 105.68) (end 166.11 105.88) (width 0.2) (layer "F.Cu") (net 2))
 (segment (start 132.231 128.599) (end 159.087686 128.599) (width 0.2) (layer "F.Cu") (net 2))
 (segment (start 163.67 84.1475) (end 166.0975 86.575) (width 0.2) (layer "F.Cu") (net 2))
 (segment (start 159.149686 128.661) (end 161.354184 128.661) (width 0.2) (layer "F.Cu") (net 2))
 (segment (start 123.01 82.67) (end 121.7 83.98) (width 0.2) (layer "F.Cu") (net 2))
 (segment (start 147.0475 105.5625) (end 146.96 105.65) (width 0.2) (layer "F.Cu") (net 2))
 (segment (start 166.0975 69.623874) (end 161.183626 64.71) (width 0.2) (layer "F.Cu") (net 2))
 (segment (start 165.295184 124.72) (end 166.08 124.72) (width 0.2) (layer "F.Cu") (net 2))
 (segment (start 163.67 74.816374) (end 163.67 84.1475) (width 0.2) (layer "F.Cu") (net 2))
 (segment (start 119.24 72.9559) (end 119.24 73.79) (width 0.2) (layer "F.Cu") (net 2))
 (via (at 119.24 73.79) (size 0.6) (drill 0.3) (layers "F.Cu" "B.Cu") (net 2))
 (via (at 122.079995 75.723437) (size 0.6) (drill 0.3) (layers "F.Cu" "B.Cu") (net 2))
 (segment (start 119.24 73.79) (end 120.146558 73.79) (width 0.2) (layer "B.Cu") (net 2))
 (segment (start 120.146558 73.79) (end 122.079995 75.723437) (width 0.2) (layer "B.Cu") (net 2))
 (segment (start 126.671 125.569) (end 126.49 125.75) (width 0.2) (layer "F.Cu") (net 3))
 (segment (start 123.34 128.45) (end 121.54 130.25) (width 0.2) (layer "F.Cu") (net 3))
 (segment (start 130.66 126.67) (end 129.559 125.569) (width 0.2) (layer "F.Cu") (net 3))
 (segment (start 123.34 128.31) (end 123.34 128.45) (width 0.2) (layer "F.Cu") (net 3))
 (segment (start 129.559 125.569) (end 126.671 125.569) (width 0.2) (layer "F.Cu") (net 3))
 (via (at 126.49 125.75) (size 0.6) (drill 0.3) (layers "F.Cu" "B.Cu") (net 3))
 (via (at 123.34 128.31) (size 0.6) (drill 0.3) (layers "F.Cu" "B.Cu") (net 3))
 (segment (start 126.49 125.75) (end 123.93 128.31) (width 0.2) (layer "B.Cu") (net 3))
 (segment (start 123.93 128.31) (end 123.34 128.31) (width 0.2) (layer "B.Cu") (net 3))
 (segment (start 121.06 127.23) (end 121.54 126.75) (width 0.2) (layer "F.Cu") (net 4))
 (segment (start 127.43 72.23) (end 128.58 73.38) (width 0.2) (layer "F.Cu") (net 4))
 (segment (start 124.24 83.98) (end 121.54 86.68) (width 0.2) (layer "F.Cu") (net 4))
 (segment (start 121.06 128.08) (end 121.06 127.23) (width 0.2) (layer "F.Cu") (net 4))
 (segment (start 121.54 86.68) (end 121.54 126.75) (width 0.2) (layer "F.Cu") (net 4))
 (segment (start 127.81 126.67) (end 127.25 127.23) (width 0.2) (layer "F.Cu") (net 4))
 (segment (start 121.26 73.33) (end 122.36 72.23) (width 0.2) (layer "F.Cu") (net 4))
 (segment (start 129.52 75.57) (end 128.58 74.63) (width 0.2) (layer "F.Cu") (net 4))
 (segment (start 121.26 73.33) (end 124.24 76.31) (width 0.2) (layer "F.Cu") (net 4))
 (segment (start 128.58 74.63) (end 128.58 73.38) (width 0.2) (layer "F.Cu") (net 4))
 (segment (start 122.36 72.23) (end 127.43 72.23) (width 0.2) (layer "F.Cu") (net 4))
 (segment (start 124.24 76.31) (end 124.24 83.98) (width 0.2) (layer "F.Cu") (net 4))
 (segment (start 128.91 126.67) (end 127.81 126.67) (width 0.2) (layer "F.Cu") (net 4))
 (via (at 129.52 75.57) (size 0.6) (drill 0.3) (layers "F.Cu" "B.Cu") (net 4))
 (via (at 127.25 127.23) (size 0.6) (drill 0.3) (layers "F.Cu" "B.Cu") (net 4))
 (via (at 121.06 128.08) (size 0.6) (drill 0.3) (layers "F.Cu" "B.Cu") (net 4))
 (segment (start 121.34 128.08) (end 121.06 128.08) (width 0.2) (layer "B.Cu") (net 4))
 (segment (start 160.57 62.17) (end 156.967 65.773) (width 0.2) (layer "B.Cu") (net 4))
 (segment (start 156.967 65.773) (end 139.317 65.773) (width 0.2) (layer "B.Cu") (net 4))
 (segment (start 139.317 65.773) (end 129.52 75.57) (width 0.2) (layer "B.Cu") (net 4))
 (segment (start 125.569 128.911) (end 122.171 128.911) (width 0.2) (layer "B.Cu") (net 4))
 (segment (start 122.171 128.911) (end 121.58 128.32) (width 0.2) (layer "B.Cu") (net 4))
 (segment (start 121.58 128.32) (end 121.34 128.08) (width 0.2) (layer "B.Cu") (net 4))
 (segment (start 127.25 127.23) (end 125.569 128.911) (width 0.2) (layer "B.Cu") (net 4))
 (segment (start 125.391 75.711) (end 125.391 126.651) (width 0.2) (layer "F.Cu") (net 1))
 (segment (start 123.01 73.33) (end 125.391 75.711) (width 0.2) (layer "F.Cu") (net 1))
 (segment (start 125.391 126.651) (end 128.91 130.17) (width 0.2) (layer "F.Cu") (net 1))
 (segment (start 120.534 76.104) (end 120.534 72.229) (width 0.2) (layer "F.Cu") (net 6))
 (segment (start 128.779 71.829) (end 130.33 73.38) (width 0.2) (layer "F.Cu") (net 6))
 (segment (start 121.26 76.83) (end 120.534 76.104) (width 0.2) (layer "F.Cu") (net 6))
 (segment (start 120.934 71.829) (end 128.779 71.829) (width 0.2) (layer "F.Cu") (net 6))
 (segment (start 120.534 72.229) (end 120.934 71.829) (width 0.2) (layer "F.Cu") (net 6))
 (segment (start 145.35631 73.393) (end 144.4201 73.393) (width 0.2) (layer "B.Cu") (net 13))
 (segment (start 141.092 69.668) (end 126.78 83.98) (width 0.2) (layer "B.Cu") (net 13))
 (segment (start 143.492 70.254957) (end 142.905043 69.668) (width 0.2) (layer "B.Cu") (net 13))
 (segment (start 145.33 77.41) (end 146.393 76.347) (width 0.2) (layer "B.Cu") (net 13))
 (segment (start 143.492 72.4649) (end 143.492 70.254957) (width 0.2) (layer "B.Cu") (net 13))
 (segment (start 144.4201 73.393) (end 143.492 72.4649) (width 0.2) (layer "B.Cu") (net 13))
 (segment (start 146.393 76.347) (end 146.393 74.42969) (width 0.2) (layer "B.Cu") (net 13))
 (segment (start 142.905043 69.668) (end 141.092 69.668) (width 0.2) (layer "B.Cu") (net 13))
 (segment (start 146.393 74.42969) (end 145.35631 73.393) (width 0.2) (layer "B.Cu") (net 13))
 (segment (start 129.32 82.990057) (end 129.32 83.98) (width 0.2) (layer "B.Cu") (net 12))
 (segment (start 145.33 74.87) (end 143.091 72.631) (width 0.2) (layer "B.Cu") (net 12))
 (segment (start 142.241057 70.069) (end 129.32 82.990057) (width 0.2) (layer "B.Cu") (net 12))
 (segment (start 142.738943 70.069) (end 142.241057 70.069) (width 0.2) (layer "B.Cu") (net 12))
 (segment (start 143.091 72.631) (end 143.091 70.421057) (width 0.2) (layer "B.Cu") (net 12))
 (segment (start 143.091 70.421057) (end 142.738943 70.069) (width 0.2) (layer "B.Cu") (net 12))
 (segment (start 160.57 74.87) (end 158.3465 77.0935) (width 0.2) (layer "F.Cu") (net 15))
 (segment (start 150.74 97.301814) (end 150.74 126.32) (width 0.2) (layer "F.Cu") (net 15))
 (segment (start 151.68 127.26) (end 159.73 127.26) (width 0.2) (layer "F.Cu") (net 15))
 (segment (start 158.3465 89.695314) (end 150.74 97.301814) (width 0.2) (layer "F.Cu") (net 15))
 (segment (start 158.3465 77.0935) (end 158.3465 89.695314) (width 0.2) (layer "F.Cu") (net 15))
 (segment (start 161.405 74.87) (end 160.57 74.87) (width 0.2) (layer "F.Cu") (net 15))
 (segment (start 150.74 126.32) (end 151.68 127.26) (width 0.2) (layer "F.Cu") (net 15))
 (segment (start 150.74 126.32) (end 150.74 126.66) (width 0.2) (layer "F.Cu") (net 15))
 (segment (start 159.76 108.22) (end 161.1485 106.8315) (width 0.2) (layer "B.Cu") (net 16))
 (segment (start 161.1485 106.8315) (end 161.1485 78.33481) (width 0.2) (layer "B.Cu") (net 16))
 (segment (start 161.1485 78.33481) (end 161.633 77.85031) (width 0.2) (layer "B.Cu") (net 16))
 (segment (start 161.633 73.393) (end 160.57 72.33) (width 0.2) (layer "B.Cu") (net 16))
 (segment (start 161.633 77.85031) (end 161.633 73.393) (width 0.2) (layer "B.Cu") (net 16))
 (segment (start 149.09003 90.454) (end 140.61 98.93403) (width 0.2) (layer "B.Cu") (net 17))
 (segment (start 140.61 98.93403) (end 140.61 108.19) (width 0.2) (layer "B.Cu") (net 17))
 (segment (start 160.57 69.79) (end 149.09003 81.26997) (width 0.2) (layer "B.Cu") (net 17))
 (segment (start 149.09003 81.26997) (end 149.09003 90.454) (width 0.2) (layer "B.Cu") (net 17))
 (segment (start 140.6975 89.0954) (end 140.6975 89.115) (width 0.2) (layer "B.Cu") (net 11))
 (segment (start 149.4171 72.33) (end 150.031 72.9439) (width 0.2) (layer "B.Cu") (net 11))
 (segment (start 150.031 72.9439) (end 150.031 79.7619) (width 0.2) (layer "B.Cu") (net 11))
 (segment (start 145.33 72.33) (end 149.4171 72.33) (width 0.2) (layer "B.Cu") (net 11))
 (segment (start 150.031 79.7619) (end 140.6975 89.0954) (width 0.2) (layer "B.Cu") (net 11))
 (segment (start 160.57 77.41) (end 160.57 88.2925) (width 0.2) (layer "B.Cu") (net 14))
 (segment (start 160.57 88.2925) (end 159.7475 89.115) (width 0.2) (layer "B.Cu") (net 14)))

